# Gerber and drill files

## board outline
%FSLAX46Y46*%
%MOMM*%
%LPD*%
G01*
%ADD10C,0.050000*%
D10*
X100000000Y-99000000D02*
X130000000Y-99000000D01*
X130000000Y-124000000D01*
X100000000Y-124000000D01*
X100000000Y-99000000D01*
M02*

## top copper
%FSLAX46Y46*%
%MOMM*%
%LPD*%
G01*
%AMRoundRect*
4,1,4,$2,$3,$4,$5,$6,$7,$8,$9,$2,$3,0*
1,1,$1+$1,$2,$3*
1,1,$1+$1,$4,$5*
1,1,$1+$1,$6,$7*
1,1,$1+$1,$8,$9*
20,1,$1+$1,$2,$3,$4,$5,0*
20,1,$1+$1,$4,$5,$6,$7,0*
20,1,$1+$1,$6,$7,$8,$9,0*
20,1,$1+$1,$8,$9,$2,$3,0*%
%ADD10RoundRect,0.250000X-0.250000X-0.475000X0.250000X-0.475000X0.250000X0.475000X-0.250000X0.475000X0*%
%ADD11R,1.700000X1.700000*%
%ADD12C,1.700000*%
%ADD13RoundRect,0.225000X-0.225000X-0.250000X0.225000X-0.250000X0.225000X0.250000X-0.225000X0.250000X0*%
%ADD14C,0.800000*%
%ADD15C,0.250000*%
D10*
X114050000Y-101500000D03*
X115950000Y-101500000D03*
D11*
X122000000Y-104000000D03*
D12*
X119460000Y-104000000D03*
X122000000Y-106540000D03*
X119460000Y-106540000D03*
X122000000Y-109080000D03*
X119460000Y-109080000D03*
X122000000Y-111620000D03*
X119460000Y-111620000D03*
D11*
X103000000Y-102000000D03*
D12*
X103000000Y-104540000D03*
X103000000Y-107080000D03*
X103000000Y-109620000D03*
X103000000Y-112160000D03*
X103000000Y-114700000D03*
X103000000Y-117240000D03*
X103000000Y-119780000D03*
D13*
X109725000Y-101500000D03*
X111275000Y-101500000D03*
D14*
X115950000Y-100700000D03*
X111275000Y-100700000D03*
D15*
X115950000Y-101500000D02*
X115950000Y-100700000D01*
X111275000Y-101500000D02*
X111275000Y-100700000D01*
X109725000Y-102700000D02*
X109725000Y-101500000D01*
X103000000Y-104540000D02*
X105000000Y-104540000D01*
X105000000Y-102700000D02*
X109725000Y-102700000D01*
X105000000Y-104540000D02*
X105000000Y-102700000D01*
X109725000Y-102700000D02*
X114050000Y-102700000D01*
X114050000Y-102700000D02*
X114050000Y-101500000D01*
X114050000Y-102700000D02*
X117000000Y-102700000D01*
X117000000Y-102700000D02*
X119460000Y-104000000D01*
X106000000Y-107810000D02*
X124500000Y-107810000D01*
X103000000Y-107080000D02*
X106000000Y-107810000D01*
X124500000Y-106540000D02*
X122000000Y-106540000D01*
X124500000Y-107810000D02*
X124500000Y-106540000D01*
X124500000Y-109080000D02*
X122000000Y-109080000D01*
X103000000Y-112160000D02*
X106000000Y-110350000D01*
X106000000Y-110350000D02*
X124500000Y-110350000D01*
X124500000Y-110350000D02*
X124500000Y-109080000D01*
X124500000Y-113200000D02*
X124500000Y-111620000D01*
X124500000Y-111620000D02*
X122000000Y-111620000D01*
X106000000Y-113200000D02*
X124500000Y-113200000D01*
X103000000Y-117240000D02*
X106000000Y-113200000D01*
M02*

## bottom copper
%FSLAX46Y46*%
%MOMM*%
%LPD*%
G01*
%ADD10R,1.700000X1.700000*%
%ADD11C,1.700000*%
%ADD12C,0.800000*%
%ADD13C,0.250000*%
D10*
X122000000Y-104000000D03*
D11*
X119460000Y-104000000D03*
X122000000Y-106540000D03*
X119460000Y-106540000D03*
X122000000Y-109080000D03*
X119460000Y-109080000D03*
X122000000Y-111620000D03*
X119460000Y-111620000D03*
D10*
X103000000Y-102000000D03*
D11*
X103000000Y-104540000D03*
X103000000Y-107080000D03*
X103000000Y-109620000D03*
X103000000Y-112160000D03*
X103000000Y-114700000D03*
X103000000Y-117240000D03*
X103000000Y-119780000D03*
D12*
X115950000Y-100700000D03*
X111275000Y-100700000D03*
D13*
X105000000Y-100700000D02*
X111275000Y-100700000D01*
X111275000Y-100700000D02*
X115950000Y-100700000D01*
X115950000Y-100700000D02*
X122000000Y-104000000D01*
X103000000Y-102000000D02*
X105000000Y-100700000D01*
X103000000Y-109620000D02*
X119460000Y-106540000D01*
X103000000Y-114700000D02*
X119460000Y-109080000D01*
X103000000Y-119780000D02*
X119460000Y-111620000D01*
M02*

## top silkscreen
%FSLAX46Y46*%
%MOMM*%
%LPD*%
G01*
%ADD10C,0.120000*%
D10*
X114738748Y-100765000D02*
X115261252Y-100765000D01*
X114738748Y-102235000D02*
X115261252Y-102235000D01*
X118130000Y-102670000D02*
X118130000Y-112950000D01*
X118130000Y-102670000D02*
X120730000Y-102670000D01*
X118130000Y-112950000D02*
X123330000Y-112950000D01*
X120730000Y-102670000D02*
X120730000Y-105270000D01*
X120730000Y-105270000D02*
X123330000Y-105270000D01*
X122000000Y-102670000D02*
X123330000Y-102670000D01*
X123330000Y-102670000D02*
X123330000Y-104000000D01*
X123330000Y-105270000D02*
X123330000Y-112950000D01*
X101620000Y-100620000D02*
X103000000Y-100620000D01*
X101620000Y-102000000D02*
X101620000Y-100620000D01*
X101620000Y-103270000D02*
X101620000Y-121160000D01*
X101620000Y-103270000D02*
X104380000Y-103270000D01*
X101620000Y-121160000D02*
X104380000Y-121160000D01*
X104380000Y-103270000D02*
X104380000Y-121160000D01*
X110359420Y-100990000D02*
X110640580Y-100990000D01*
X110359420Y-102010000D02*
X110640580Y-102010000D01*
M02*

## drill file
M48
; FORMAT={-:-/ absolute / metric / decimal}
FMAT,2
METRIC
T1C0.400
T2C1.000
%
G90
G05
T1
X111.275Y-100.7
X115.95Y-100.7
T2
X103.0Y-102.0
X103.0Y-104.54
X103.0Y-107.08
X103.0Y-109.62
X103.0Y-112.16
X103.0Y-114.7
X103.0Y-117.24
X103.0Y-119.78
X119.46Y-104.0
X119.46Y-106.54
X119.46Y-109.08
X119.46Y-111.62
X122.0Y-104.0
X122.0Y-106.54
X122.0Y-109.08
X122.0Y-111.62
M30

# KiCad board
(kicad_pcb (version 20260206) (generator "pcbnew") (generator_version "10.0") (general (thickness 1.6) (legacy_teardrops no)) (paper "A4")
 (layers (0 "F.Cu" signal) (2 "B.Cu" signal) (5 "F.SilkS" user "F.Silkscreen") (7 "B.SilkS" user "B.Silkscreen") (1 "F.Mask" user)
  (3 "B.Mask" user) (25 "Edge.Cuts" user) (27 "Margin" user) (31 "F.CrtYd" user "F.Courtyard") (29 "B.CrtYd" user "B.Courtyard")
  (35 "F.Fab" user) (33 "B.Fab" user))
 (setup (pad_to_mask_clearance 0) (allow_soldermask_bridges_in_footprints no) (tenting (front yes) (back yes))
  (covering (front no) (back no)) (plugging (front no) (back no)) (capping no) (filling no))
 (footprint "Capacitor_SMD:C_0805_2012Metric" (layer "F.Cu") (at 115 101.5)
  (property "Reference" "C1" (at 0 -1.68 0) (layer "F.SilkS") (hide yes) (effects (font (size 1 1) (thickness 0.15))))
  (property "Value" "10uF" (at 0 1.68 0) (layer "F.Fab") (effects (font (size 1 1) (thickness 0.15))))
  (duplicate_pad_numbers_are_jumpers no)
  (fp_line (start -0.261252 -0.735) (end 0.261252 -0.735) (stroke (width 0.12) (type solid)) (layer "F.SilkS"))
  (fp_line (start -0.261252 0.735) (end 0.261252 0.735) (stroke (width 0.12) (type solid)) (layer "F.SilkS"))
  (pad "1" smd roundrect (at -0.95 0) (size 1 1.45) (layers "F.Cu" "F.Mask" "F.Paste") (roundrect_rratio 0.25) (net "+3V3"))
  (pad "2" smd roundrect (at 0.95 0) (size 1 1.45) (layers "F.Cu" "F.Mask" "F.Paste") (roundrect_rratio 0.25) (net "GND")))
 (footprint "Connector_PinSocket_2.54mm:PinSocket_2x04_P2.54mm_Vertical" (layer "F.Cu") (at 122 104)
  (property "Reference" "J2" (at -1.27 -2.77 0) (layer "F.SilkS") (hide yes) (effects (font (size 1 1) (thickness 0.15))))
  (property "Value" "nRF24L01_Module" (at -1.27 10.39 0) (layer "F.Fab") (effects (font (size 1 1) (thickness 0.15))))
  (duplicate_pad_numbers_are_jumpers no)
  (fp_line (start -3.87 -1.33) (end -3.87 8.95) (stroke (width 0.12) (type solid)) (layer "F.SilkS"))
  (fp_line (start -3.87 -1.33) (end -1.27 -1.33) (stroke (width 0.12) (type solid)) (layer "F.SilkS"))
  (fp_line (start -3.87 8.95) (end 1.33 8.95) (stroke (width 0.12) (type solid)) (layer "F.SilkS"))
  (fp_line (start -1.27 -1.33) (end -1.27 1.27) (stroke (width 0.12) (type solid)) (layer "F.SilkS"))
  (fp_line (start -1.27 1.27) (end 1.33 1.27) (stroke (width 0.12) (type solid)) (layer "F.SilkS"))
  (fp_line (start 0 -1.33) (end 1.33 -1.33) (stroke (width 0.12) (type solid)) (layer "F.SilkS"))
  (fp_line (start 1.33 -1.33) (end 1.33 0) (stroke (width 0.12) (type solid)) (layer "F.SilkS"))
  (fp_line (start 1.33 1.27) (end 1.33 8.95) (stroke (width 0.12) (type solid)) (layer "F.SilkS"))
  (pad "1" thru_hole rect (at 0 0) (size 1.7 1.7) (drill 1) (layers "*.Cu" "*.Mask") (remove_unused_layers no) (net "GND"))
  (pad "2" thru_hole circle (at -2.54 0) (size 1.7 1.7) (drill 1) (layers "*.Cu" "*.Mask") (remove_unused_layers no) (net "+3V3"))
  (pad "3" thru_hole circle (at 0 2.54) (size 1.7 1.7) (drill 1) (layers "*.Cu" "*.Mask") (remove_unused_layers no) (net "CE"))
  (pad "4" thru_hole circle (at -2.54 2.54) (size 1.7 1.7) (drill 1) (layers "*.Cu" "*.Mask") (remove_unused_layers no) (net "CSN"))
  (pad "5" thru_hole circle (at 0 5.08) (size 1.7 1.7) (drill 1) (layers "*.Cu" "*.Mask") (remove_unused_layers no) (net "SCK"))
  (pad "6" thru_hole circle (at -2.54 5.08) (size 1.7 1.7) (drill 1) (layers "*.Cu" "*.Mask") (remove_unused_layers no) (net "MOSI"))
  (pad "7" thru_hole circle (at 0 7.62) (size 1.7 1.7) (drill 1) (layers "*.Cu" "*.Mask") (remove_unused_layers no) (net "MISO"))
  (pad "8" thru_hole circle (at -2.54 7.62) (size 1.7 1.7) (drill 1) (layers "*.Cu" "*.Mask") (remove_unused_layers no) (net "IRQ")))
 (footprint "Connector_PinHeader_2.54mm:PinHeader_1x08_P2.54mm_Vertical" (layer "F.Cu") (at 103 102)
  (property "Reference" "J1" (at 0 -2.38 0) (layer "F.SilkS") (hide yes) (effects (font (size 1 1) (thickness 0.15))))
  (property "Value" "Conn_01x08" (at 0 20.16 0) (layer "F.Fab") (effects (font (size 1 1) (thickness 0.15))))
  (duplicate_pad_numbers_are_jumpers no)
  (fp_line (start -1.38 -1.38) (end 0 -1.38) (stroke (width 0.12) (type solid)) (layer "F.SilkS"))
  (fp_line (start -1.38 0) (end -1.38 -1.38) (stroke (width 0.12) (type solid)) (layer "F.SilkS"))
  (fp_line (start -1.38 1.27) (end -1.38 19.16) (stroke (width 0.12) (type solid)) (layer "F.SilkS"))
  (fp_line (start -1.38 1.27) (end 1.38 1.27) (stroke (width 0.12) (type solid)) (layer "F.SilkS"))
  (fp_line (start -1.38 19.16) (end 1.38 19.16) (stroke (width 0.12) (type solid)) (layer "F.SilkS"))
  (fp_line (start 1.38 1.27) (end 1.38 19.16) (stroke (width 0.12) (type solid)) (layer "F.SilkS"))
  (pad "1" thru_hole rect (at 0 0) (size 1.7 1.7) (drill 1) (layers "*.Cu" "*.Mask") (remove_unused_layers no) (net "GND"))
  (pad "2" thru_hole circle (at 0 2.54) (size 1.7 1.7) (drill 1) (layers "*.Cu" "*.Mask") (remove_unused_layers no) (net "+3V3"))
  (pad "3" thru_hole circle (at 0 5.08) (size 1.7 1.7) (drill 1) (layers "*.Cu" "*.Mask") (remove_unused_layers no) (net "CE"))
  (pad "4" thru_hole circle (at 0 7.62) (size 1.7 1.7) (drill 1) (layers "*.Cu" "*.Mask") (remove_unused_layers no) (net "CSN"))
  (pad "5" thru_hole circle (at 0 10.16) (size 1.7 1.7) (drill 1) (layers "*.Cu" "*.Mask") (remove_unused_layers no) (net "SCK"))
  (pad "6" thru_hole circle (at 0 12.7) (size 1.7 1.7) (drill 1) (layers "*.Cu" "*.Mask") (remove_unused_layers no) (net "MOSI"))
  (pad "7" thru_hole circle (at 0 15.24) (size 1.7 1.7) (drill 1) (layers "*.Cu" "*.Mask") (remove_unused_layers no) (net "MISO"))
  (pad "8" thru_hole circle (at 0 17.78) (size 1.7 1.7) (drill 1) (layers "*.Cu" "*.Mask") (remove_unused_layers no) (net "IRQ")))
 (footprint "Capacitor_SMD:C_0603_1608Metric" (layer "F.Cu") (at 110.5 101.5)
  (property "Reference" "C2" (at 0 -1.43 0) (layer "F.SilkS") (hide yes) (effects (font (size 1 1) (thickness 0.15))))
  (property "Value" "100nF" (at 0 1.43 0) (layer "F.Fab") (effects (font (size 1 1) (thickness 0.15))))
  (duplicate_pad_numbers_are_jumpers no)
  (fp_line (start -0.14058 -0.51) (end 0.14058 -0.51) (stroke (width 0.12) (type solid)) (layer "F.SilkS"))
  (fp_line (start -0.14058 0.51) (end 0.14058 0.51) (stroke (width 0.12) (type solid)) (layer "F.SilkS"))
  (pad "1" smd roundrect (at -0.775 0) (size 0.9 0.95) (layers "F.Cu" "F.Mask" "F.Paste") (roundrect_rratio 0.25) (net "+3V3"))
  (pad "2" smd roundrect (at 0.775 0) (size 0.9 0.95) (layers "F.Cu" "F.Mask" "F.Paste") (roundrect_rratio 0.25) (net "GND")))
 (gr_rect (start 100 99) (end 130 124) (stroke (width 0.05) (type default)) (fill no) (layer "Edge.Cuts"))
 (segment (start 115.95 101.5) (end 115.95 100.7) (width 0.25) (layer "F.Cu") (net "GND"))
 (segment (start 111.275 101.5) (end 111.275 100.7) (width 0.25) (layer "F.Cu") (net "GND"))
 (via (at 115.95 100.7) (size 0.8) (drill 0.4) (layers "F.Cu" "B.Cu") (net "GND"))
 (via (at 111.275 100.7) (size 0.8) (drill 0.4) (layers "F.Cu" "B.Cu") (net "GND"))
 (segment (start 105 100.7) (end 111.275 100.7) (width 0.25) (layer "B.Cu") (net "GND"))
 (segment (start 111.275 100.7) (end 115.95 100.7) (width 0.25) (layer "B.Cu") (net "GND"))
 (segment (start 115.95 100.7) (end 122 104) (width 0.25) (layer "B.Cu") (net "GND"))
 (segment (start 103 102) (end 105 100.7) (width 0.25) (layer "B.Cu") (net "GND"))
 (segment (start 109.725 102.7) (end 109.725 101.5) (width 0.25) (layer "F.Cu") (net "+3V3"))
 (segment (start 103 104.54) (end 105 104.54) (width 0.25) (layer "F.Cu") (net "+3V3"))
 (segment (start 105 102.7) (end 109.725 102.7) (width 0.25) (layer "F.Cu") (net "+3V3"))
 (segment (start 105 104.54) (end 105 102.7) (width 0.25) (layer "F.Cu") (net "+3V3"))
 (segment (start 109.725 102.7) (end 114.05 102.7) (width 0.25) (layer "F.Cu") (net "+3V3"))
 (segment (start 114.05 102.7) (end 114.05 101.5) (width 0.25) (layer "F.Cu") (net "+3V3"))
 (segment (start 114.05 102.7) (end 117 102.7) (width 0.25) (layer "F.Cu") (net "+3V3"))
 (segment (start 117 102.7) (end 119.46 104) (width 0.25) (layer "F.Cu") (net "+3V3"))
 (segment (start 106 107.81) (end 124.5 107.81) (width 0.25) (layer "F.Cu") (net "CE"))
 (segment (start 103 107.08) (end 106 107.81) (width 0.25) (layer "F.Cu") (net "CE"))
 (segment (start 124.5 106.54) (end 122 106.54) (width 0.25) (layer "F.Cu") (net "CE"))
 (segment (start 124.5 107.81) (end 124.5 106.54) (width 0.25) (layer "F.Cu") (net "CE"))
 (segment (start 103 109.62) (end 119.46 106.54) (width 0.25) (layer "B.Cu") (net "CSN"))
 (segment (start 124.5 109.08) (end 122 109.08) (width 0.25) (layer "F.Cu") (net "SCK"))
 (segment (start 103 112.16) (end 106 110.35) (width 0.25) (layer "F.Cu") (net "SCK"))
 (segment (start 106 110.35) (end 124.5 110.35) (width 0.25) (layer "F.Cu") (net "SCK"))
 (segment (start 124.5 110.35) (end 124.5 109.08) (width 0.25) (layer "F.Cu") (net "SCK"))
 (segment (start 103 114.7) (end 119.46 109.08) (width 0.25) (layer "B.Cu") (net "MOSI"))
 (segment (start 124.5 113.2) (end 124.5 111.62) (width 0.25) (layer "F.Cu") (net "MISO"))
 (segment (start 124.5 111.62) (end 122 111.62) (width 0.25) (layer "F.Cu") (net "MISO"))
 (segment (start 106 113.2) (end 124.5 113.2) (width 0.25) (layer "F.Cu") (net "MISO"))
 (segment (start 103 117.24) (end 106 113.2) (width 0.25) (layer "F.Cu") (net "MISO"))
 (segment (start 103 119.78) (end 119.46 111.62) (width 0.25) (layer "B.Cu") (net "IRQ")))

